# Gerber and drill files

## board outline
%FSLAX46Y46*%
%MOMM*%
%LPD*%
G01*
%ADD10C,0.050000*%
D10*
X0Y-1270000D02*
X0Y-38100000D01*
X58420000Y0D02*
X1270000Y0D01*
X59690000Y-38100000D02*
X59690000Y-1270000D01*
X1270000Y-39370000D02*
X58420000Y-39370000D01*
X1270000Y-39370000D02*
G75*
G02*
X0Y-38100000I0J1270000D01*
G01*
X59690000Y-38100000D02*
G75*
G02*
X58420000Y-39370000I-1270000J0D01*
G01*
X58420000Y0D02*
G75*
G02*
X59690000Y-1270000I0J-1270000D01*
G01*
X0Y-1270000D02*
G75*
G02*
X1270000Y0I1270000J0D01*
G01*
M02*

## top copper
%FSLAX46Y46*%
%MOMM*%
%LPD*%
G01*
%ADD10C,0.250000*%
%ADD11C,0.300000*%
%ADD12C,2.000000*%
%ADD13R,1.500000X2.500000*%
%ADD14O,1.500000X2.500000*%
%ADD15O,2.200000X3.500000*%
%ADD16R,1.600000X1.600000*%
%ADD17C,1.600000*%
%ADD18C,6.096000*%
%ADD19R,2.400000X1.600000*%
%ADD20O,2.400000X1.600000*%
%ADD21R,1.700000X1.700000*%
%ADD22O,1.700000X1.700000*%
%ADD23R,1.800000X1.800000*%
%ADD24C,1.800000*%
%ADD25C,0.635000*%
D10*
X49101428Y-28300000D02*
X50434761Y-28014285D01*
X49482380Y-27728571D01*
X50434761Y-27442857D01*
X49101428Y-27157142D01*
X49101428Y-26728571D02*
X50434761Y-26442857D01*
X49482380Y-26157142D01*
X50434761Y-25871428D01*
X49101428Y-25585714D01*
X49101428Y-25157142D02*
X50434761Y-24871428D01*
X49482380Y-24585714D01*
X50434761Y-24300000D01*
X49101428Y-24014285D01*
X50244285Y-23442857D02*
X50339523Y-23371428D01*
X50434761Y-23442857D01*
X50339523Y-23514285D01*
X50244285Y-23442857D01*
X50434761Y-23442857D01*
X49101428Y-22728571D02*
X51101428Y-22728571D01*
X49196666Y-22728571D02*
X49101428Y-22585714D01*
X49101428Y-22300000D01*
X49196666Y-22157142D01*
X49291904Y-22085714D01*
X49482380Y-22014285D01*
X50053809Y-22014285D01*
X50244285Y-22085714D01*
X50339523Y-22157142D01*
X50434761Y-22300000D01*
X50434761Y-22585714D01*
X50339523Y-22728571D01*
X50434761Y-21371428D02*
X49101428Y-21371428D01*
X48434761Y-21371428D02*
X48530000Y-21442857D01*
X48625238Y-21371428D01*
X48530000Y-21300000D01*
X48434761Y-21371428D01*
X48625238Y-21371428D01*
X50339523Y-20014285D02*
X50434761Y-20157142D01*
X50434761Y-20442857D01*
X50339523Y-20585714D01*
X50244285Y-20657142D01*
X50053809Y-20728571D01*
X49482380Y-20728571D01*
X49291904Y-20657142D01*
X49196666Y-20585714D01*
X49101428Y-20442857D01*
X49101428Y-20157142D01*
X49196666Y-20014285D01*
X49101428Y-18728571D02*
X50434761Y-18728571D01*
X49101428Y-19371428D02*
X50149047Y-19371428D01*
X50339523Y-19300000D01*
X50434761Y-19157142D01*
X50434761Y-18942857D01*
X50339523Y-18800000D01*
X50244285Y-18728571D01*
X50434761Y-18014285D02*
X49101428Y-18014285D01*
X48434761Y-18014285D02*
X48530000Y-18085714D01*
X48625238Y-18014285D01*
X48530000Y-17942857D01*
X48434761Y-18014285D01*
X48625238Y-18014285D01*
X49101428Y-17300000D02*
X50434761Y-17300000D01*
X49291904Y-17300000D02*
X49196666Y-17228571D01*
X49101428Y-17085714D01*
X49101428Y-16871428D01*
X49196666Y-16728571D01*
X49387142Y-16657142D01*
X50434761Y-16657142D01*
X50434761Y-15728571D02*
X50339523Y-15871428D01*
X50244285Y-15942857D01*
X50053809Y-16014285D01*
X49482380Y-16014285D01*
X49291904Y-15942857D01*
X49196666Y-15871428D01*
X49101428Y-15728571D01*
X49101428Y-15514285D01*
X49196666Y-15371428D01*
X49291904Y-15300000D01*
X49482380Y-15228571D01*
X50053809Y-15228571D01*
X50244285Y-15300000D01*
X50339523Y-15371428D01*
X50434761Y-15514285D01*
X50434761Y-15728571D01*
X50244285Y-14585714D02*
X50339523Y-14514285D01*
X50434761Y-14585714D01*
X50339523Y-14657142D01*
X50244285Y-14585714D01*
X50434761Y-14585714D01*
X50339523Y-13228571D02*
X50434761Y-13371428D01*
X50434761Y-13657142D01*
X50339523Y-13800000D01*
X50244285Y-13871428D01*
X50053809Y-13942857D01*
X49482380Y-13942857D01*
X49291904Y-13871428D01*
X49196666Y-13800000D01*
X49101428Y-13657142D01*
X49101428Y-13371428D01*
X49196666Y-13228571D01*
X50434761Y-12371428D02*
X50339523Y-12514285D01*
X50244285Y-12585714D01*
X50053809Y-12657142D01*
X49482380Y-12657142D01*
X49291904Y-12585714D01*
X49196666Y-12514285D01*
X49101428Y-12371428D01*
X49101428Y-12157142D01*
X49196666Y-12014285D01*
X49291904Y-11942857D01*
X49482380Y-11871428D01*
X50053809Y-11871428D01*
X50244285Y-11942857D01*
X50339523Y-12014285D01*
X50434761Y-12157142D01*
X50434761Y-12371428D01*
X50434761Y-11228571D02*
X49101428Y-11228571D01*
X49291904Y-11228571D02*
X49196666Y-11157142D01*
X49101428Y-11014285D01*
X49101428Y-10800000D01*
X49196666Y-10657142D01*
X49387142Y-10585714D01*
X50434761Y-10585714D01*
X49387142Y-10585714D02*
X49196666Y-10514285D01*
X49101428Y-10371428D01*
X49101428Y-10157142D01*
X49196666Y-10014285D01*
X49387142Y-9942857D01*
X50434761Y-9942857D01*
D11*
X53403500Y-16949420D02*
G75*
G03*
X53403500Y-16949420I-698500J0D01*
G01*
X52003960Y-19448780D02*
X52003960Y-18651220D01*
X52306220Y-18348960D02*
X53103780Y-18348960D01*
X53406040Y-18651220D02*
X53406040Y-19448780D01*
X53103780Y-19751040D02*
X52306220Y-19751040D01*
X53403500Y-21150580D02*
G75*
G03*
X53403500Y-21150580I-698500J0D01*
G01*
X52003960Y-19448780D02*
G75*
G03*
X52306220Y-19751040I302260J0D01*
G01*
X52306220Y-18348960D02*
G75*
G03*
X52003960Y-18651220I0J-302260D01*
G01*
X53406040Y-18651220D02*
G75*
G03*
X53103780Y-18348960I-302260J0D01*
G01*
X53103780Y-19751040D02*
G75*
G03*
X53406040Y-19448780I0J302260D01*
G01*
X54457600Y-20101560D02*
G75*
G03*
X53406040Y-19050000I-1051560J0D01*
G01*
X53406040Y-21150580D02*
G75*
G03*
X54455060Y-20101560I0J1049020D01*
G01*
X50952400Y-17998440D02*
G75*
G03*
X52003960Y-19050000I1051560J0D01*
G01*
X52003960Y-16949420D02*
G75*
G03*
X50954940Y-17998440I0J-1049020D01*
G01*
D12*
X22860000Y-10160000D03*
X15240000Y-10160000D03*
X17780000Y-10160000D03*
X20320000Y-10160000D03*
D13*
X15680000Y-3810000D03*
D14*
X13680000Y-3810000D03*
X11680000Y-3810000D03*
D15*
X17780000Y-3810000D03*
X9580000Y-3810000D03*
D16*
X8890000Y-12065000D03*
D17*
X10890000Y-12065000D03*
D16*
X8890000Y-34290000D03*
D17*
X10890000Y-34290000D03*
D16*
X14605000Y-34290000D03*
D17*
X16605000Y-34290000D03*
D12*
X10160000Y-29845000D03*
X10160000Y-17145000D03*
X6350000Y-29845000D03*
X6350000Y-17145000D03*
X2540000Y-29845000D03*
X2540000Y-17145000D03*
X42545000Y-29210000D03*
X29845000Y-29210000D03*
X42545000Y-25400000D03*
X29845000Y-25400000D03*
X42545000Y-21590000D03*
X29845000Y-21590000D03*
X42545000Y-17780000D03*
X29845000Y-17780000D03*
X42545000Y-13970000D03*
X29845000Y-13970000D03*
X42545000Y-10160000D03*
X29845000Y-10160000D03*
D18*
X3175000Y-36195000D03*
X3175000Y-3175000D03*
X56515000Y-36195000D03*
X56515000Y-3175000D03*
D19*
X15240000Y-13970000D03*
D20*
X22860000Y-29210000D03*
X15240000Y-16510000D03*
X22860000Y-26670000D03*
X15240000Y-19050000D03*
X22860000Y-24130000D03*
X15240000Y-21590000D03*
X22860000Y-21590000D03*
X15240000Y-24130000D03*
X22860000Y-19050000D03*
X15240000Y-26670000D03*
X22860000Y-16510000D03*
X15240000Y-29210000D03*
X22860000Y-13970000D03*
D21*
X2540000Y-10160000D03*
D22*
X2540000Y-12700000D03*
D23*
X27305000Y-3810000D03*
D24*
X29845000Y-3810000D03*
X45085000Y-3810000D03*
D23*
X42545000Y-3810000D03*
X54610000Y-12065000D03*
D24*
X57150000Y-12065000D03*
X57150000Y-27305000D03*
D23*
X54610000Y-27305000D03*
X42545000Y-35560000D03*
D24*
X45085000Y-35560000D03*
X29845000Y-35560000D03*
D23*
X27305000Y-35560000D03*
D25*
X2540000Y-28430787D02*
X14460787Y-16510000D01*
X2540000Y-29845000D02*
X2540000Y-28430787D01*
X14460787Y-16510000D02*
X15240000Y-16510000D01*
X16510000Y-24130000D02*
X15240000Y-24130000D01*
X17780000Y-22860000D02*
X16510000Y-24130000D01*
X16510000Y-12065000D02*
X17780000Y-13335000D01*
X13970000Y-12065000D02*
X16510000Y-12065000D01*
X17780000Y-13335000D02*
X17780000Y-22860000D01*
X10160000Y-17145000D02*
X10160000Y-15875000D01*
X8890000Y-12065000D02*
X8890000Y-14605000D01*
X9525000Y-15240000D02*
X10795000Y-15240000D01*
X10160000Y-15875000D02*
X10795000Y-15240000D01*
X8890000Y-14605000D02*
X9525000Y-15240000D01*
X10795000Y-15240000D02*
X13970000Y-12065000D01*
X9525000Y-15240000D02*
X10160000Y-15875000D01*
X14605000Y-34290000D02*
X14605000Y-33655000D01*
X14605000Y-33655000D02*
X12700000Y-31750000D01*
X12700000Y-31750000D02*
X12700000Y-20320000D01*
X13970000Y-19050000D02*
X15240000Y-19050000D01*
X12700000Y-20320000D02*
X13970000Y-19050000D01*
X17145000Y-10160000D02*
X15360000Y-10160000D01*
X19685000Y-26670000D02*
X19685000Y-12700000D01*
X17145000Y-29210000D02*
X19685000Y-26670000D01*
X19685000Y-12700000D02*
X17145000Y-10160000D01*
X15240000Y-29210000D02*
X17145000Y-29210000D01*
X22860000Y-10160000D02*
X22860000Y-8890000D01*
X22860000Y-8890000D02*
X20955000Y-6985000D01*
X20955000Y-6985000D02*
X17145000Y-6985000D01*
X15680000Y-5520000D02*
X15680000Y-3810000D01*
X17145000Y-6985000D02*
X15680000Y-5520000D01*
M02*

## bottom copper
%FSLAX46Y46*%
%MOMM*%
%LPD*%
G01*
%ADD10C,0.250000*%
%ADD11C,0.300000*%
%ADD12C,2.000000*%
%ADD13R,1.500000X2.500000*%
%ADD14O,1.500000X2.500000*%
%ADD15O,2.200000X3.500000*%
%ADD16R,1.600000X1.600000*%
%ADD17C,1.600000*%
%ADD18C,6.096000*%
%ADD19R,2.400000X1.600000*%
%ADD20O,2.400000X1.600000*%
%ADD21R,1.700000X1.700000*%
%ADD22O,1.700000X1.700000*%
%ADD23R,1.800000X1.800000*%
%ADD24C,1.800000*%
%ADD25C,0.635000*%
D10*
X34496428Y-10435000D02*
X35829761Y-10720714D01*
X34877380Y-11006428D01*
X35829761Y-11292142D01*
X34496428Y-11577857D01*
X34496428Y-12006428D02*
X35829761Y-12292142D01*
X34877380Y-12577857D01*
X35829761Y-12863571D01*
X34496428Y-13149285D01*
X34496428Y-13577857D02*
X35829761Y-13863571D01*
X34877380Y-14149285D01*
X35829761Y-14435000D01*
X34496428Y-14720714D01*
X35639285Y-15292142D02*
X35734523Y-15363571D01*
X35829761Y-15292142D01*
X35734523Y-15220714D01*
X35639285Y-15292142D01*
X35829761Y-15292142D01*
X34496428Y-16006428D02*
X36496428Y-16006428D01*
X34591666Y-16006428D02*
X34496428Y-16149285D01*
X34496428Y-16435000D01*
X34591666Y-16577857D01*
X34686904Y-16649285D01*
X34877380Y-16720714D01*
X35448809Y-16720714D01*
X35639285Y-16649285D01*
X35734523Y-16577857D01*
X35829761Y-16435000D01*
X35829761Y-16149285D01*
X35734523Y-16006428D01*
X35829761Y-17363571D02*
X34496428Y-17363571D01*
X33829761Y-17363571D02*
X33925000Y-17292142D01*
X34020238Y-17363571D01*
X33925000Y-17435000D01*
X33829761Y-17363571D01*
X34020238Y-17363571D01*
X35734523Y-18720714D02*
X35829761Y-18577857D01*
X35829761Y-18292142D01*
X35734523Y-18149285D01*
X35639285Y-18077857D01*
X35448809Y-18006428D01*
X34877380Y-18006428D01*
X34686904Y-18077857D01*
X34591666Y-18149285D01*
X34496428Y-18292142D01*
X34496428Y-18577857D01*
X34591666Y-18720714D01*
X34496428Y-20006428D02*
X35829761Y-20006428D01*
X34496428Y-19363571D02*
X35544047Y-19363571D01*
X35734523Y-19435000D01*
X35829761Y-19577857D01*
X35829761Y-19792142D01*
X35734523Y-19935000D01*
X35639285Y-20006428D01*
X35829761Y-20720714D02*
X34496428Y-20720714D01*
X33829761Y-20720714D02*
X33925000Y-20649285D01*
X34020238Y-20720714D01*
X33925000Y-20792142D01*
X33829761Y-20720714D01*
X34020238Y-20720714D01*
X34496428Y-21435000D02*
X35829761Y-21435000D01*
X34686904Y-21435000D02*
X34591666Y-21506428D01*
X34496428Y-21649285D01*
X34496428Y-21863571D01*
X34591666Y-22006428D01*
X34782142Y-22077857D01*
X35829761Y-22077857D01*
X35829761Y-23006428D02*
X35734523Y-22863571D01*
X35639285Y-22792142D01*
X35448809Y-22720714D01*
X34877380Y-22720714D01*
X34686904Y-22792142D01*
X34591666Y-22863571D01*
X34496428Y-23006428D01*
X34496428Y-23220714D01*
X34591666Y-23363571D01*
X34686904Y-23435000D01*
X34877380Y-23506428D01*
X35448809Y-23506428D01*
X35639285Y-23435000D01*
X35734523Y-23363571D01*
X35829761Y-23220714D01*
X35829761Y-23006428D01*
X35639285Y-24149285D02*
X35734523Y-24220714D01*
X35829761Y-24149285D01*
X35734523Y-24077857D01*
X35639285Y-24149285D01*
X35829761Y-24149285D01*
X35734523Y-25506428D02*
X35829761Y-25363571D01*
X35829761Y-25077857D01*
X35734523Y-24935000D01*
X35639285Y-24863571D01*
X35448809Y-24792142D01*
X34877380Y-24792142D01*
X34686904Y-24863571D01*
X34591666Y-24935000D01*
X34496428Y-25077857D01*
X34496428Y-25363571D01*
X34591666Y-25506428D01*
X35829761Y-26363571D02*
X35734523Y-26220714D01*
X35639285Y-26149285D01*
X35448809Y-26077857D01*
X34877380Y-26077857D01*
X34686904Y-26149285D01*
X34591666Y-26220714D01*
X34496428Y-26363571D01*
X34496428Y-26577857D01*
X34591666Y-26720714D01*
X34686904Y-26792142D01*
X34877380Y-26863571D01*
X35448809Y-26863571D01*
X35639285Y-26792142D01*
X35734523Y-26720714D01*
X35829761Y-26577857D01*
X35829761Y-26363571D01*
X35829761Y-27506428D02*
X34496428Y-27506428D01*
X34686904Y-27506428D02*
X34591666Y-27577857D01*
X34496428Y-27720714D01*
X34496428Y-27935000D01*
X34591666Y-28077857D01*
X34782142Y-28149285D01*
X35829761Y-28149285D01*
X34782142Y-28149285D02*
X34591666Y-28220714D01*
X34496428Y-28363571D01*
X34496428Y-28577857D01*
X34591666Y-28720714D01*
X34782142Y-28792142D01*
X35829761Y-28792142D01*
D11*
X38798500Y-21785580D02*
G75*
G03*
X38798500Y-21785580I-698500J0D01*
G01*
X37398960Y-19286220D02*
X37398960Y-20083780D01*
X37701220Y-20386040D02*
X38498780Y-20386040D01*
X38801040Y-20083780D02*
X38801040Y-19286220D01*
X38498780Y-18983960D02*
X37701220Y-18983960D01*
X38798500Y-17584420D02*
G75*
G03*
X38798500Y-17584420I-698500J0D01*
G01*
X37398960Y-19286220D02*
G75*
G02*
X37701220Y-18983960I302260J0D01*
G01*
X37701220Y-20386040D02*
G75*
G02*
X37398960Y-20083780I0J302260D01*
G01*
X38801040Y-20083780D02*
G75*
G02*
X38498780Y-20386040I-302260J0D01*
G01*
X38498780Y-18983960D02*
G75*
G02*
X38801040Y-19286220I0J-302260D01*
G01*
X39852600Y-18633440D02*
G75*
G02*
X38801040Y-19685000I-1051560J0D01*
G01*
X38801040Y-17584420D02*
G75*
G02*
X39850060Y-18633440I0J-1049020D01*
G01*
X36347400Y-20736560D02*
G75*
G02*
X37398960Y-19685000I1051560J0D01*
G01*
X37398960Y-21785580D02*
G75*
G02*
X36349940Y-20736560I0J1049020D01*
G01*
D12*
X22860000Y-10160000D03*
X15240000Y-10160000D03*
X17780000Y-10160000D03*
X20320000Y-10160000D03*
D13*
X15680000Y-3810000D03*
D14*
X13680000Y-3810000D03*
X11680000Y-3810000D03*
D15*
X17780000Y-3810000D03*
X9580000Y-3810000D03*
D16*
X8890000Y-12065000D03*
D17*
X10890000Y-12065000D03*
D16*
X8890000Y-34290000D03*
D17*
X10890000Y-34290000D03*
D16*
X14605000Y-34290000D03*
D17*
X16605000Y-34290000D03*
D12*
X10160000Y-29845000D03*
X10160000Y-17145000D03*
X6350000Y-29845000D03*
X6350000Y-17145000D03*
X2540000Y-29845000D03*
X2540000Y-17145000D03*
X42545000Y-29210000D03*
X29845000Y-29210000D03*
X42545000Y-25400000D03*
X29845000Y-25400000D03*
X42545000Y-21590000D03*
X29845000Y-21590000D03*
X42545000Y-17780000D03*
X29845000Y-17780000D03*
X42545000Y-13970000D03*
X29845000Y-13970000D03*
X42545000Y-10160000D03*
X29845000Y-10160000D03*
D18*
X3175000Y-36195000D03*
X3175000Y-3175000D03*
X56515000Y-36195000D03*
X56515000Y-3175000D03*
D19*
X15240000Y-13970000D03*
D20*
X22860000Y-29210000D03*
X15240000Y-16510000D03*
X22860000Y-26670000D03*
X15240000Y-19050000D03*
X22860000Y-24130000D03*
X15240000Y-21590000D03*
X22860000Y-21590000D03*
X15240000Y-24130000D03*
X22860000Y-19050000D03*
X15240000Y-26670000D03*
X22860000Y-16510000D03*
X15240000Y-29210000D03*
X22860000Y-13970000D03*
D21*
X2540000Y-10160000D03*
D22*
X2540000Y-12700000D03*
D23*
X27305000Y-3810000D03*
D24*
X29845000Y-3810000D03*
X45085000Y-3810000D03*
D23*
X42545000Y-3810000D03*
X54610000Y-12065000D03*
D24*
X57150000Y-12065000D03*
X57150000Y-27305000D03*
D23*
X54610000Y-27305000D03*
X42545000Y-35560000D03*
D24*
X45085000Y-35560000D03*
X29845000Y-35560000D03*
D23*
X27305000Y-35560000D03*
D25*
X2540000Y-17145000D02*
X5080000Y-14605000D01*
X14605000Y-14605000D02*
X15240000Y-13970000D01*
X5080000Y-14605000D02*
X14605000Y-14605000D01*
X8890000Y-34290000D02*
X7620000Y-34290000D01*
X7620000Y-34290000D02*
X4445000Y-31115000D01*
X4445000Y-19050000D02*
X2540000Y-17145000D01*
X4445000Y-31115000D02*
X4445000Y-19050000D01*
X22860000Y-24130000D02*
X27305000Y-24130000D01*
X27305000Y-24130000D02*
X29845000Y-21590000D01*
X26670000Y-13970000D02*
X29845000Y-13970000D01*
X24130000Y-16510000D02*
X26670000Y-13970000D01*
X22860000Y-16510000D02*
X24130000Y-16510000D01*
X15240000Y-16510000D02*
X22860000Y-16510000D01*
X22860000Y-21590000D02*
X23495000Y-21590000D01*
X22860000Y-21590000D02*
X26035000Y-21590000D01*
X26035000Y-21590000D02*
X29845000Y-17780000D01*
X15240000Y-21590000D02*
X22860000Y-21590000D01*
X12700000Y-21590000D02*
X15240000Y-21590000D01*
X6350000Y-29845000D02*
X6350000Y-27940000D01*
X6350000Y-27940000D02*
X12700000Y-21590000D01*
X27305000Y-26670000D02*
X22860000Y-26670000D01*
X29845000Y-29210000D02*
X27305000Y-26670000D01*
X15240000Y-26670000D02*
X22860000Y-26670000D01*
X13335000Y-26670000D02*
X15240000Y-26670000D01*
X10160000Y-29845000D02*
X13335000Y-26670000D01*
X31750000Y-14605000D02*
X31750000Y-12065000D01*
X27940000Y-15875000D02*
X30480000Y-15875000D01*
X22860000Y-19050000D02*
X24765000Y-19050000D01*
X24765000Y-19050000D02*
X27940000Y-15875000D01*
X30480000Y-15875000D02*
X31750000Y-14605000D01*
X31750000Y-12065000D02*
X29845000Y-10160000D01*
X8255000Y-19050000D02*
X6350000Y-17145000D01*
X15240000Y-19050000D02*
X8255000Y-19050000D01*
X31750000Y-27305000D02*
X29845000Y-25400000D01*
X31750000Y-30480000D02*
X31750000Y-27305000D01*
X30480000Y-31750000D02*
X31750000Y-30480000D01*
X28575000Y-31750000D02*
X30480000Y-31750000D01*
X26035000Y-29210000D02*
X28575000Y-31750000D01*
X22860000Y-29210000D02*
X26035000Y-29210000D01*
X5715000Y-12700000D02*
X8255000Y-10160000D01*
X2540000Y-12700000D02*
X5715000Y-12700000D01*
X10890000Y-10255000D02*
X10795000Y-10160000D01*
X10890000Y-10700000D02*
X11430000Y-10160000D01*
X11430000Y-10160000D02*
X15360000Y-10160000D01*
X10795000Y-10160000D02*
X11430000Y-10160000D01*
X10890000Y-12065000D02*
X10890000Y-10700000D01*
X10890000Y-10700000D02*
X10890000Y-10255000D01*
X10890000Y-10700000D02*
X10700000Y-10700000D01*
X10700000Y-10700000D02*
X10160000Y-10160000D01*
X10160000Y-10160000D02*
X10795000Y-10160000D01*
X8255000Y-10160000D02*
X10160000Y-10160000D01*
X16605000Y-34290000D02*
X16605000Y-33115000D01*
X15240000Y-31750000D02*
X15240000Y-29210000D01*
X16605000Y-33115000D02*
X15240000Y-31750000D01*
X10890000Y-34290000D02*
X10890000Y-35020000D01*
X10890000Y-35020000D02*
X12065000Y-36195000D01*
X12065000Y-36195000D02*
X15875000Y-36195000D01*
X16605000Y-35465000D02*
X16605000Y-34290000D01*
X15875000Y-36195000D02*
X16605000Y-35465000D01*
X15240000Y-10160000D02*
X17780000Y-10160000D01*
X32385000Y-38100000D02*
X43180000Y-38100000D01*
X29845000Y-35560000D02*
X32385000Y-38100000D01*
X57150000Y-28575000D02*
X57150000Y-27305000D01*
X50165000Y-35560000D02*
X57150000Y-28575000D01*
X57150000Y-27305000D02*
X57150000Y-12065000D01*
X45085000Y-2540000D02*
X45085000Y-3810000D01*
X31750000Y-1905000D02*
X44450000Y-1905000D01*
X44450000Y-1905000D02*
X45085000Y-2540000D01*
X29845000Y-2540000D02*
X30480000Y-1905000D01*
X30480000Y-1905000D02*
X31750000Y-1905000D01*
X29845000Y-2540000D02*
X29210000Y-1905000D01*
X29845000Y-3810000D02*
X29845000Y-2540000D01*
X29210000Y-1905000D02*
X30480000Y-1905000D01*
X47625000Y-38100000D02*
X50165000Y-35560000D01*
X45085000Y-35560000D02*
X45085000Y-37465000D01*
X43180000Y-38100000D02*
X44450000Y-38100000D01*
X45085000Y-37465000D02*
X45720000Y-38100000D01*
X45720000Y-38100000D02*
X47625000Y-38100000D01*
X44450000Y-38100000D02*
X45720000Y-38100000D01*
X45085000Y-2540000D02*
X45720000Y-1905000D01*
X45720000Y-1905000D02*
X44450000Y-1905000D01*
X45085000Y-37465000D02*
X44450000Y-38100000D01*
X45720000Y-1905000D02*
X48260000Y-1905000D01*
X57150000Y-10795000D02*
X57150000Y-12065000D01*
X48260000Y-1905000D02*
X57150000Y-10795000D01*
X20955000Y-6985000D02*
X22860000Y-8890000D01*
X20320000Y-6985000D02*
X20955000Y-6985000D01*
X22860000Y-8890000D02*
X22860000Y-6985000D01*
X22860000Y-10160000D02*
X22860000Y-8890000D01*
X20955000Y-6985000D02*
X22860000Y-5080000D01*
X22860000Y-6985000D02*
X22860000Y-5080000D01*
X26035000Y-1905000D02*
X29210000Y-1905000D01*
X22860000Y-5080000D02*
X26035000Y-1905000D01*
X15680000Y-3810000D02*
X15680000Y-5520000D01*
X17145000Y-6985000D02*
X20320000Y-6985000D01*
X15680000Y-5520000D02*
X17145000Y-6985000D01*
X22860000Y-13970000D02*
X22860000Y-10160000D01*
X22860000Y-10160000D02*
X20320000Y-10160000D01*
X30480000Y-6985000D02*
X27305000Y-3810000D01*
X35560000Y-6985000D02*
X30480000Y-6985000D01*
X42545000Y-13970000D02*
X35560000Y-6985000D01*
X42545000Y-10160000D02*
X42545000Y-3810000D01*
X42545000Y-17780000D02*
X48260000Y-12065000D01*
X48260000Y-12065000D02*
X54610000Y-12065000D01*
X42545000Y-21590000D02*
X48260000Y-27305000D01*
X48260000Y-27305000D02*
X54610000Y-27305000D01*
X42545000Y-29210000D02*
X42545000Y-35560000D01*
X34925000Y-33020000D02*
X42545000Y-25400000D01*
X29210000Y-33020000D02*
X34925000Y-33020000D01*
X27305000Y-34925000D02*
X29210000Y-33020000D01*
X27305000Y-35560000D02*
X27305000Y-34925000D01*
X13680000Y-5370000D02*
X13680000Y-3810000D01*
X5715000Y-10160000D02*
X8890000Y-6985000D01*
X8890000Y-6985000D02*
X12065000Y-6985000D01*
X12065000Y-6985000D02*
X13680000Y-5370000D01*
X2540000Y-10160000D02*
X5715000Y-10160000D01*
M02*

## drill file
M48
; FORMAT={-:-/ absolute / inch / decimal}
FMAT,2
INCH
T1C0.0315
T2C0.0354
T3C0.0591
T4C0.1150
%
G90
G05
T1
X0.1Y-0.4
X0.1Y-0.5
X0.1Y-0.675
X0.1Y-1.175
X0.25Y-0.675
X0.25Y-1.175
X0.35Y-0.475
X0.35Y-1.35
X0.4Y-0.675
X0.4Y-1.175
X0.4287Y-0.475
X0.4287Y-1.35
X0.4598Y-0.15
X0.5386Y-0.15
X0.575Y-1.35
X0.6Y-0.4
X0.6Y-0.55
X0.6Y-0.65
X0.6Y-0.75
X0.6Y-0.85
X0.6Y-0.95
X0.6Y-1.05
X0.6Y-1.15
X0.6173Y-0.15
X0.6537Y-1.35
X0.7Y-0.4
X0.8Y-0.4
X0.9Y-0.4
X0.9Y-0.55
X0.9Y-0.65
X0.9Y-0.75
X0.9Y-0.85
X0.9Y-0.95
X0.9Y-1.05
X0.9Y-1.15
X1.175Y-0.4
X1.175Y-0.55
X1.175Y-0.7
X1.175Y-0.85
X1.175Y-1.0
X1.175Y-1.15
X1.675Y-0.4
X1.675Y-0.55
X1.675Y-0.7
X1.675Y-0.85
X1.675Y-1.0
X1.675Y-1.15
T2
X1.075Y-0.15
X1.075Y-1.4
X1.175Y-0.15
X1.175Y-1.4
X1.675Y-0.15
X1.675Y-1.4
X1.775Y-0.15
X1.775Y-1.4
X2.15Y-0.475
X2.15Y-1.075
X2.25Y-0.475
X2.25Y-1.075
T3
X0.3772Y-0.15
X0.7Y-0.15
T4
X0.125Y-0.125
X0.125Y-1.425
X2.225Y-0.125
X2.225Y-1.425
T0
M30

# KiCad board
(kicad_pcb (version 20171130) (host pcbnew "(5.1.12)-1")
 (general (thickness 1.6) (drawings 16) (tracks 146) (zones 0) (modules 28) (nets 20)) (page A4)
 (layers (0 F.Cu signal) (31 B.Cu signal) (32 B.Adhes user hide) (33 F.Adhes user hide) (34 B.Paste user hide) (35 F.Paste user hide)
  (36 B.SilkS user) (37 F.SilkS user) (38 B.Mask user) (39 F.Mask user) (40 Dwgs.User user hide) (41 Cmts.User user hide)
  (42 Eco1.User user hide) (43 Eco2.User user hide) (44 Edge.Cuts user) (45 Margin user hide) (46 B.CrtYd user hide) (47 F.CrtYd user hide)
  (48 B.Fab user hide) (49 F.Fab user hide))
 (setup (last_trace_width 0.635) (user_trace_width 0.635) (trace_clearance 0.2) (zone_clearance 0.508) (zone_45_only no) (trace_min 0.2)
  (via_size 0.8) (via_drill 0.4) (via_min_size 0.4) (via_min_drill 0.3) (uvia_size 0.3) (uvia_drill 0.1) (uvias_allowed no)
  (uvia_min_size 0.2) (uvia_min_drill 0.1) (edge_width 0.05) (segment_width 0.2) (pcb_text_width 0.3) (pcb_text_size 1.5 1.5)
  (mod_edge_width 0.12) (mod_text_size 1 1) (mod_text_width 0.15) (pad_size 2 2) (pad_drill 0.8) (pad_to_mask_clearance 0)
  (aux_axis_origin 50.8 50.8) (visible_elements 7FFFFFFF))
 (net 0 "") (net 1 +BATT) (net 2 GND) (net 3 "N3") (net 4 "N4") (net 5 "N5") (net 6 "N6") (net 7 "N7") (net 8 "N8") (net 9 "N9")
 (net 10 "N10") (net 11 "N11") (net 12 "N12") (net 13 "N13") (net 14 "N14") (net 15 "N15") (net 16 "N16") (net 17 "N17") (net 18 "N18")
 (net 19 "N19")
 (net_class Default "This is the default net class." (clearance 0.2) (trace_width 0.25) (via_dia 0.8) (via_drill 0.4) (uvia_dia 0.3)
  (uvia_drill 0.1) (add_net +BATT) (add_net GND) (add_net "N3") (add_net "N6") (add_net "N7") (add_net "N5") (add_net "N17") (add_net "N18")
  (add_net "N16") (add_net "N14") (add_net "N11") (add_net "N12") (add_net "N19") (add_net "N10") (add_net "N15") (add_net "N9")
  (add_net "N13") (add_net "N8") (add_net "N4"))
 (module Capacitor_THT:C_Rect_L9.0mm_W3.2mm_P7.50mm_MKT (layer F.Cu) (at 73.66 60.96 180)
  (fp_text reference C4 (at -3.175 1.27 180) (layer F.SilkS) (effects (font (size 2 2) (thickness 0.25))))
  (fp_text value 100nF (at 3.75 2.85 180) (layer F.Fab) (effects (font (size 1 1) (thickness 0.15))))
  (pad 1 thru_hole circle (at 0 0 180) (size 2 2) (drill 0.8) (layers *.Cu *.Mask) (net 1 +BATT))
  (pad 2 thru_hole circle (at 7.62 0 180) (size 2 2) (drill 0.8) (layers *.Cu *.Mask) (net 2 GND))
  (pad 2 thru_hole circle (at 5.08 0 180) (size 2 2) (drill 0.8) (layers *.Cu *.Mask) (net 2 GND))
  (pad 1 thru_hole circle (at 2.54 0 180) (size 2 2) (drill 0.8) (layers *.Cu *.Mask) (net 1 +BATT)))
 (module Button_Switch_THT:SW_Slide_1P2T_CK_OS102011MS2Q (layer F.Cu) (at 66.48 54.61 180)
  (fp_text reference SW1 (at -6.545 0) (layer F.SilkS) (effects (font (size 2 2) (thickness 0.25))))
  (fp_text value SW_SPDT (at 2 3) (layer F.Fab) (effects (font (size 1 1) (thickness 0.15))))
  (pad 1 thru_hole rect (at 0 0 180) (size 1.5 2.5) (drill 0.8) (layers *.Cu *.Mask) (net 1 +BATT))
  (pad 2 thru_hole oval (at 2 0 180) (size 1.5 2.5) (drill 0.8) (layers *.Cu *.Mask) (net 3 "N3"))
  (pad 3 thru_hole oval (at 4 0 180) (size 1.5 2.5) (drill 0.8) (layers *.Cu *.Mask) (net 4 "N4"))
  (pad "" thru_hole oval (at -2.1 0 180) (size 2.2 3.5) (drill 1.5) (layers *.Cu *.Mask))
  (pad "" thru_hole oval (at 6.1 0 180) (size 2.2 3.5) (drill 1.5) (layers *.Cu *.Mask)))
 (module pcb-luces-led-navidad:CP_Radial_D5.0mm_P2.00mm (layer F.Cu) (at 59.69 62.865)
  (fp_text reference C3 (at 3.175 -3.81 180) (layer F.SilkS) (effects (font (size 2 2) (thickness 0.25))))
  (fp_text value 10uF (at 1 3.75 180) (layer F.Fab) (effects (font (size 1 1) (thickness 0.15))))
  (pad 1 thru_hole rect (at 0 0) (size 1.6 1.6) (drill 0.8) (layers *.Cu *.Mask) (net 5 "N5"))
  (pad 2 thru_hole circle (at 2 0) (size 1.6 1.6) (drill 0.8) (layers *.Cu *.Mask) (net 2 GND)))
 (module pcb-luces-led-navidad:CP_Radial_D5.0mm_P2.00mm (layer F.Cu) (at 59.69 85.09)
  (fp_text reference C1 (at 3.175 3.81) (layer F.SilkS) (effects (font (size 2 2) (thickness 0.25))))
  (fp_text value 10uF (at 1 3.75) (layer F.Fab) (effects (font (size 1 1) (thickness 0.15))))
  (pad 1 thru_hole rect (at 0 0) (size 1.6 1.6) (drill 0.8) (layers *.Cu *.Mask) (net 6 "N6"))
  (pad 2 thru_hole circle (at 2 0) (size 1.6 1.6) (drill 0.8) (layers *.Cu *.Mask) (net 2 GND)))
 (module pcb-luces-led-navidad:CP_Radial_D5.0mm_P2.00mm (layer F.Cu) (at 65.405 85.09)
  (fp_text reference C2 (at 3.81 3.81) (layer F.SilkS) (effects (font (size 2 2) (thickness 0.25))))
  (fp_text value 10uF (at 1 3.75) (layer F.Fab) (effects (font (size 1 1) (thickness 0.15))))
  (pad 1 thru_hole rect (at 0 0) (size 1.6 1.6) (drill 0.8) (layers *.Cu *.Mask) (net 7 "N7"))
  (pad 2 thru_hole circle (at 2 0) (size 1.6 1.6) (drill 0.8) (layers *.Cu *.Mask) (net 2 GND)))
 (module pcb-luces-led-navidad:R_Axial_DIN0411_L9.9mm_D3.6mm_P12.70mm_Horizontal (layer F.Cu) (at 60.96 80.645 90)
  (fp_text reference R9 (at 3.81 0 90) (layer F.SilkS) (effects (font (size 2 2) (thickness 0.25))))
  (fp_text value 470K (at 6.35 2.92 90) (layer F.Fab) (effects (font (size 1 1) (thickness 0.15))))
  (pad 1 thru_hole circle (at 0 0 90) (size 2 2) (drill 0.8) (layers *.Cu *.Mask) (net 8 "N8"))
  (pad 2 thru_hole circle (at 12.7 0 90) (size 2 2) (drill 0.8) (layers *.Cu *.Mask) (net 5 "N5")))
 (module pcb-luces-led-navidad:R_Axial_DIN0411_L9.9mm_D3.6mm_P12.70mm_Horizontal (layer F.Cu) (at 57.15 80.645 90)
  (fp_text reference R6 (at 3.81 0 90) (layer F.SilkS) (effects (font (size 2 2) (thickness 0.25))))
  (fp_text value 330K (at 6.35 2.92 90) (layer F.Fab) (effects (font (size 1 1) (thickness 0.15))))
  (pad 1 thru_hole circle (at 0 0 90) (size 2 2) (drill 0.8) (layers *.Cu *.Mask) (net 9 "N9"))
  (pad 2 thru_hole circle (at 12.7 0 90) (size 2 2) (drill 0.8) (layers *.Cu *.Mask) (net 7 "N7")))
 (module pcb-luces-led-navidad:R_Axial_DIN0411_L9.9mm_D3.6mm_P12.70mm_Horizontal (layer F.Cu) (at 53.34 80.645 90)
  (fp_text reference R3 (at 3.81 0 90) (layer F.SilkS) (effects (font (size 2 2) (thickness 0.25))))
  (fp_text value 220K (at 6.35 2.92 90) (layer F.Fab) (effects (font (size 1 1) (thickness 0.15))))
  (pad 1 thru_hole circle (at 0 0 90) (size 2 2) (drill 0.8) (layers *.Cu *.Mask) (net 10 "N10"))
  (pad 2 thru_hole circle (at 12.7 0 90) (size 2 2) (drill 0.8) (layers *.Cu *.Mask) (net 6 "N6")))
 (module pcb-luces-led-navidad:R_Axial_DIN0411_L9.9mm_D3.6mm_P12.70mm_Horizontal (layer F.Cu) (at 93.345 80.01 180)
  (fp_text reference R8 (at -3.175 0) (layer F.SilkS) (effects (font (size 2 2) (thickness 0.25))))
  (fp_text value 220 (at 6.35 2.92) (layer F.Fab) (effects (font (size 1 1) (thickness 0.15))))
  (pad 1 thru_hole circle (at 0 0 180) (size 2 2) (drill 0.8) (layers *.Cu *.Mask) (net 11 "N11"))
  (pad 2 thru_hole circle (at 12.7 0 180) (size 2 2) (drill 0.8) (layers *.Cu *.Mask) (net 8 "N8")))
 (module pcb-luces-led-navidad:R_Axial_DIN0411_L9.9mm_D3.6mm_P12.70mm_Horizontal (layer F.Cu) (at 93.345 76.2 180)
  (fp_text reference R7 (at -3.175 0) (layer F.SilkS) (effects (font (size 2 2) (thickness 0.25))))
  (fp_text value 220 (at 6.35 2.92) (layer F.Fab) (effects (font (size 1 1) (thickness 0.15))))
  (pad 1 thru_hole circle (at 0 0 180) (size 2 2) (drill 0.8) (layers *.Cu *.Mask) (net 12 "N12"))
  (pad 2 thru_hole circle (at 12.7 0 180) (size 2 2) (drill 0.8) (layers *.Cu *.Mask) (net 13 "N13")))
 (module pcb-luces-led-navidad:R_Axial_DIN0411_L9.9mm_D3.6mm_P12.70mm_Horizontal (layer F.Cu) (at 93.345 72.39 180)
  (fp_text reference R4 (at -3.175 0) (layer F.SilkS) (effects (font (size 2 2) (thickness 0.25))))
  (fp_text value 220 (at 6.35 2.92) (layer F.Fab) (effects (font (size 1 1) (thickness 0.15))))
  (pad 1 thru_hole circle (at 0 0 180) (size 2 2) (drill 0.8) (layers *.Cu *.Mask) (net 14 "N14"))
  (pad 2 thru_hole circle (at 12.7 0 180) (size 2 2) (drill 0.8) (layers *.Cu *.Mask) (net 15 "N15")))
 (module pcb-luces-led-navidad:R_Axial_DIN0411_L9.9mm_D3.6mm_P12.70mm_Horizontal (layer F.Cu) (at 93.345 68.58 180)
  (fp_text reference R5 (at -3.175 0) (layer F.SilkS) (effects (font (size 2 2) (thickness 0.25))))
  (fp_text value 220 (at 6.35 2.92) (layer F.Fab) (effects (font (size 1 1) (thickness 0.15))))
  (pad 1 thru_hole circle (at 0 0 180) (size 2 2) (drill 0.8) (layers *.Cu *.Mask) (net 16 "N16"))
  (pad 2 thru_hole circle (at 12.7 0 180) (size 2 2) (drill 0.8) (layers *.Cu *.Mask) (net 9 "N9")))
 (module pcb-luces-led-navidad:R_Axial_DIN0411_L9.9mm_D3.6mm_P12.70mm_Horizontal (layer F.Cu) (at 93.345 64.77 180)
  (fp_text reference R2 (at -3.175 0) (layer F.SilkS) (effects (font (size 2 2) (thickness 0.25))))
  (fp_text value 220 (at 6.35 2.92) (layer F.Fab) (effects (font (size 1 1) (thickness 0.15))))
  (pad 1 thru_hole circle (at 0 0 180) (size 2 2) (drill 0.8) (layers *.Cu *.Mask) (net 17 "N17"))
  (pad 2 thru_hole circle (at 12.7 0 180) (size 2 2) (drill 0.8) (layers *.Cu *.Mask) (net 10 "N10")))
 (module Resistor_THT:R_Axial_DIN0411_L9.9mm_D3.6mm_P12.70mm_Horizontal (layer F.Cu) (at 93.345 60.96 180)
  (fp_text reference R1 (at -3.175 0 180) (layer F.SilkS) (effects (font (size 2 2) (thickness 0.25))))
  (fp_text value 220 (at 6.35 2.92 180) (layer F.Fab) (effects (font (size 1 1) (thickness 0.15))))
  (pad 1 thru_hole circle (at 0 0 180) (size 2 2) (drill 0.8) (layers *.Cu *.Mask) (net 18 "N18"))
  (pad 2 thru_hole circle (at 12.7 0 180) (size 2 2) (drill 0.8) (layers *.Cu *.Mask) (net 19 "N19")))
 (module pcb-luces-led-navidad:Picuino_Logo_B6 (layer B.Cu) (at 103.505 69.85 270)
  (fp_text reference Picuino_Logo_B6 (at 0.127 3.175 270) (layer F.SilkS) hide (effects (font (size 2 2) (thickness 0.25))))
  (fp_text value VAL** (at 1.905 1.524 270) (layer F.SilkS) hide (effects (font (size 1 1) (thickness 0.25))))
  (fp_circle (center -2.10058 0) (end -1.40208 0) (layer F.Cu) (width 0.3))
  (fp_line (start 0.39878 0.70104) (end -0.39878 0.70104) (layer F.Cu) (width 0.3))
  (fp_line (start -0.70104 0.39878) (end -0.70104 -0.39878) (layer F.Cu) (width 0.3))
  (fp_line (start -0.39878 -0.70104) (end 0.39878 -0.70104) (layer F.Cu) (width 0.3))
  (fp_line (start 0.70104 -0.39878) (end 0.70104 0.39878) (layer F.Cu) (width 0.3))
  (fp_circle (center 2.10058 0) (end 2.79908 0) (layer F.Cu) (width 0.3))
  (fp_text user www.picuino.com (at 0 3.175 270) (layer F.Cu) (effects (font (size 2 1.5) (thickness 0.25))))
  (fp_arc (start 0.39878 0.39878) (end 0.70104 0.39878) (angle 90) (layer F.Cu) (width 0.3))
  (fp_arc (start -0.39878 0.39878) (end -0.39878 0.70104) (angle 90) (layer F.Cu) (width 0.3))
  (fp_arc (start -0.39878 -0.39878) (end -0.70104 -0.39878) (angle 90) (layer F.Cu) (width 0.3))
  (fp_arc (start 0.39878 -0.39878) (end 0.39878 -0.70104) (angle 90) (layer F.Cu) (width 0.3))
  (fp_arc (start 1.05156 -0.70104) (end 0 -0.70104) (angle 90) (layer F.Cu) (width 0.3))
  (fp_arc (start 1.05156 -0.70104) (end 1.05156 -1.75006) (angle 90) (layer F.Cu) (width 0.3))
  (fp_arc (start -1.05156 0.70104) (end 0 0.70104) (angle 90) (layer F.Cu) (width 0.3))
  (fp_arc (start -1.05156 0.70104) (end -1.05156 1.75006) (angle 90) (layer F.Cu) (width 0.3)))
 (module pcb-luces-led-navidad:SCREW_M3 (layer F.Cu) (at 53.975 86.995)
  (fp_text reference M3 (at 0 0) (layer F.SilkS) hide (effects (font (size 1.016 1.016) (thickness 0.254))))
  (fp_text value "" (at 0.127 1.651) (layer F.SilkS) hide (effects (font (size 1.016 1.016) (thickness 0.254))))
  (pad "" thru_hole circle (at 0 0) (size 6.096 6.096) (drill 2.921) (layers *.Cu F.SilkS)))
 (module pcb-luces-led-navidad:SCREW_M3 (layer F.Cu) (at 53.975 53.975)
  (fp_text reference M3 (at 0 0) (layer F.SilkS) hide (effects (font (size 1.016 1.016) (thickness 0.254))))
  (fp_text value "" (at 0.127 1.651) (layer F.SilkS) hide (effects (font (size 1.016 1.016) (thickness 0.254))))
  (pad "" thru_hole circle (at 0 0) (size 6.096 6.096) (drill 2.921) (layers *.Cu F.SilkS)))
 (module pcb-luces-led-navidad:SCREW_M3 (layer F.Cu) (at 107.315 86.995)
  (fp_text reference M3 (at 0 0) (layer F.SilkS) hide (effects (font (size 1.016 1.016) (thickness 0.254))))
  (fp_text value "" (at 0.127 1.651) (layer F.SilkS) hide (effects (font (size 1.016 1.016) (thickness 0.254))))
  (pad "" thru_hole circle (at 0 0) (size 6.096 6.096) (drill 2.921) (layers *.Cu F.SilkS)))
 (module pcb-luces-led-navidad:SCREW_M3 (layer F.Cu) (at 107.315 53.975)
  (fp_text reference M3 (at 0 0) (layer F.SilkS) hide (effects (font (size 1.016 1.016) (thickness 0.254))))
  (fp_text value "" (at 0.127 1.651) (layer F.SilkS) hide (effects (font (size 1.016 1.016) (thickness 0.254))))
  (pad "" thru_hole circle (at 0 0) (size 6.096 6.096) (drill 2.921) (layers *.Cu F.SilkS)))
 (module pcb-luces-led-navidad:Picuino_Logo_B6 (layer F.Cu) (at 88.9 70.485 90)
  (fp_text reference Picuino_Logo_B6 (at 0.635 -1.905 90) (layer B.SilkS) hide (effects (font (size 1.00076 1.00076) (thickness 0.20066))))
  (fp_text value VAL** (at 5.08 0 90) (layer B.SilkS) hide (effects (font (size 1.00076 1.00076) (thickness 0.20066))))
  (fp_circle (center -2.10058 0) (end -1.40208 0) (layer B.Cu) (width 0.3))
  (fp_line (start 0.39878 -0.70104) (end -0.39878 -0.70104) (layer B.Cu) (width 0.3))
  (fp_line (start -0.70104 -0.39878) (end -0.70104 0.39878) (layer B.Cu) (width 0.3))
  (fp_line (start -0.39878 0.70104) (end 0.39878 0.70104) (layer B.Cu) (width 0.3))
  (fp_line (start 0.70104 0.39878) (end 0.70104 -0.39878) (layer B.Cu) (width 0.3))
  (fp_circle (center 2.10058 0) (end 2.79908 0) (layer B.Cu) (width 0.3))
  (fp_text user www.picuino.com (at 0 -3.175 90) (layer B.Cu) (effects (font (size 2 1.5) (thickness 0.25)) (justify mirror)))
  (fp_arc (start 0.39878 -0.39878) (end 0.70104 -0.39878) (angle -90) (layer B.Cu) (width 0.3))
  (fp_arc (start -0.39878 -0.39878) (end -0.39878 -0.70104) (angle -90) (layer B.Cu) (width 0.3))
  (fp_arc (start -0.39878 0.39878) (end -0.70104 0.39878) (angle -90) (layer B.Cu) (width 0.3))
  (fp_arc (start 0.39878 0.39878) (end 0.39878 0.70104) (angle -90) (layer B.Cu) (width 0.3))
  (fp_arc (start 1.05156 0.70104) (end 0 0.70104) (angle -90) (layer B.Cu) (width 0.3))
  (fp_arc (start 1.05156 0.70104) (end 1.05156 1.75006) (angle -90) (layer B.Cu) (width 0.3))
  (fp_arc (start -1.05156 -0.70104) (end 0 -0.70104) (angle -90) (layer B.Cu) (width 0.3))
  (fp_arc (start -1.05156 -0.70104) (end -1.05156 -1.75006) (angle -90) (layer B.Cu) (width 0.3)))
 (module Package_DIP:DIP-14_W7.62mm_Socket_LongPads (layer F.Cu) (at 66.04 64.77)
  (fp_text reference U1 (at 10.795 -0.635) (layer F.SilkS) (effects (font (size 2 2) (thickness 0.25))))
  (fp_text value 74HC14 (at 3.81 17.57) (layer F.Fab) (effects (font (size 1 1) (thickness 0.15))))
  (pad 1 thru_hole rect (at 0 0) (size 2.4 1.6) (drill 0.8) (layers *.Cu *.Mask) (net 6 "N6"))
  (pad 8 thru_hole oval (at 7.62 15.24) (size 2.4 1.6) (drill 0.8) (layers *.Cu *.Mask) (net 13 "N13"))
  (pad 2 thru_hole oval (at 0 2.54) (size 2.4 1.6) (drill 0.8) (layers *.Cu *.Mask) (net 10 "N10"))
  (pad 9 thru_hole oval (at 7.62 12.7) (size 2.4 1.6) (drill 0.8) (layers *.Cu *.Mask) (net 8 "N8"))
  (pad 3 thru_hole oval (at 0 5.08) (size 2.4 1.6) (drill 0.8) (layers *.Cu *.Mask) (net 7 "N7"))
  (pad 10 thru_hole oval (at 7.62 10.16) (size 2.4 1.6) (drill 0.8) (layers *.Cu *.Mask) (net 15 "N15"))
  (pad 4 thru_hole oval (at 0 7.62) (size 2.4 1.6) (drill 0.8) (layers *.Cu *.Mask) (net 9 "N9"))
  (pad 11 thru_hole oval (at 7.62 7.62) (size 2.4 1.6) (drill 0.8) (layers *.Cu *.Mask) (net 9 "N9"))
  (pad 5 thru_hole oval (at 0 10.16) (size 2.4 1.6) (drill 0.8) (layers *.Cu *.Mask) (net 5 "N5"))
  (pad 12 thru_hole oval (at 7.62 5.08) (size 2.4 1.6) (drill 0.8) (layers *.Cu *.Mask) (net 19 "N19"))
  (pad 6 thru_hole oval (at 0 12.7) (size 2.4 1.6) (drill 0.8) (layers *.Cu *.Mask) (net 8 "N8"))
  (pad 13 thru_hole oval (at 7.62 2.54) (size 2.4 1.6) (drill 0.8) (layers *.Cu *.Mask) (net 10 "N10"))
  (pad 7 thru_hole oval (at 0 15.24) (size 2.4 1.6) (drill 0.8) (layers *.Cu *.Mask) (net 2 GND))
  (pad 14 thru_hole oval (at 7.62 0) (size 2.4 1.6) (drill 0.8) (layers *.Cu *.Mask) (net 1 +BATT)))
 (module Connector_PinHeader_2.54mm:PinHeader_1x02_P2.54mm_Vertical (layer F.Cu) (at 53.34 60.96)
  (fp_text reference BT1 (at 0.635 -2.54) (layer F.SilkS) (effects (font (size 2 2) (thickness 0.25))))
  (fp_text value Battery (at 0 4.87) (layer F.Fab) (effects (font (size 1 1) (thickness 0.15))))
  (pad 1 thru_hole rect (at 0 0) (size 1.7 1.7) (drill 0.8) (layers *.Cu *.Mask) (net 3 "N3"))
  (pad 2 thru_hole oval (at 0 2.54) (size 1.7 1.7) (drill 0.8) (layers *.Cu *.Mask) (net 2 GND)))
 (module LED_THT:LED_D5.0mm (layer F.Cu) (at 78.105 54.61)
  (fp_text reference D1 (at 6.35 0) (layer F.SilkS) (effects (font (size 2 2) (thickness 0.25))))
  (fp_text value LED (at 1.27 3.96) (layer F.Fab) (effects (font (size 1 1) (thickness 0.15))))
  (pad 1 thru_hole rect (at 0 0) (size 1.8 1.8) (drill 0.9) (layers *.Cu *.Mask) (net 17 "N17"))
  (pad 2 thru_hole circle (at 2.54 0) (size 1.8 1.8) (drill 0.9) (layers *.Cu *.Mask) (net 1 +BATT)))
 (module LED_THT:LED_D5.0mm (layer F.Cu) (at 93.345 54.61)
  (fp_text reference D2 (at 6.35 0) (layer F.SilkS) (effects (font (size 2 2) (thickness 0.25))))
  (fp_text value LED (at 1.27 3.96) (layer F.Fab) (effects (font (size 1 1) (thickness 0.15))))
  (pad 2 thru_hole circle (at 2.54 0) (size 1.8 1.8) (drill 0.9) (layers *.Cu *.Mask) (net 1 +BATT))
  (pad 1 thru_hole rect (at 0 0) (size 1.8 1.8) (drill 0.9) (layers *.Cu *.Mask) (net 18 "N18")))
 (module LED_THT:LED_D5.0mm (layer F.Cu) (at 105.41 62.865)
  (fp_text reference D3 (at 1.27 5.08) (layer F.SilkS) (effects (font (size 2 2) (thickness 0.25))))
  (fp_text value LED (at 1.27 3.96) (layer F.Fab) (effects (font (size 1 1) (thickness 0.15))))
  (pad 1 thru_hole rect (at 0 0) (size 1.8 1.8) (drill 0.9) (layers *.Cu *.Mask) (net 16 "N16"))
  (pad 2 thru_hole circle (at 2.54 0) (size 1.8 1.8) (drill 0.9) (layers *.Cu *.Mask) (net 1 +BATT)))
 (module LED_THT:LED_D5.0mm (layer F.Cu) (at 105.41 78.105)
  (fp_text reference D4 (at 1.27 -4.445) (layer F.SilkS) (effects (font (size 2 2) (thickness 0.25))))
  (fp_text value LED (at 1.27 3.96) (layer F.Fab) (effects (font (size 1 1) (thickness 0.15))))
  (pad 2 thru_hole circle (at 2.54 0) (size 1.8 1.8) (drill 0.9) (layers *.Cu *.Mask) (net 1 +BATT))
  (pad 1 thru_hole rect (at 0 0) (size 1.8 1.8) (drill 0.9) (layers *.Cu *.Mask) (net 14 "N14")))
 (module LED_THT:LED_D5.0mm (layer F.Cu) (at 93.345 86.36)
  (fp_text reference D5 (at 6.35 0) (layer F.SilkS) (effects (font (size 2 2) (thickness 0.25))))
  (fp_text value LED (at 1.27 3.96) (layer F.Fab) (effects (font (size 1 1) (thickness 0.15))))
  (pad 1 thru_hole rect (at 0 0) (size 1.8 1.8) (drill 0.9) (layers *.Cu *.Mask) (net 11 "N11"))
  (pad 2 thru_hole circle (at 2.54 0) (size 1.8 1.8) (drill 0.9) (layers *.Cu *.Mask) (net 1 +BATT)))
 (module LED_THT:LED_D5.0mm (layer F.Cu) (at 78.105 86.36)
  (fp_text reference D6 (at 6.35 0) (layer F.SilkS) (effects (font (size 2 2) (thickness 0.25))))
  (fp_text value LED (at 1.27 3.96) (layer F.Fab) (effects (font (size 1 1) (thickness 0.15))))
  (pad 2 thru_hole circle (at 2.54 0) (size 1.8 1.8) (drill 0.9) (layers *.Cu *.Mask) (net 1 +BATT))
  (pad 1 thru_hole rect (at 0 0) (size 1.8 1.8) (drill 0.9) (layers *.Cu *.Mask) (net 12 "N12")))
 (gr_line (start 50.8 52.07) (end 50.8 88.9) (layer Edge.Cuts) (width 0.05))
 (gr_line (start 109.22 50.8) (end 52.07 50.8) (layer Edge.Cuts) (width 0.05))
 (gr_line (start 110.49 88.9) (end 110.49 52.07) (layer Edge.Cuts) (width 0.05))
 (gr_line (start 52.07 90.17) (end 109.22 90.17) (layer Edge.Cuts) (width 0.05))
 (gr_arc (start 52.07 88.9) (end 50.8 88.9) (angle -90) (layer Edge.Cuts) (width 0.05))
 (gr_arc (start 109.22 88.9) (end 109.22 90.17) (angle -90) (layer Edge.Cuts) (width 0.05))
 (gr_arc (start 109.22 52.07) (end 110.49 52.07) (angle -90) (layer Edge.Cuts) (width 0.05))
 (gr_arc (start 52.07 52.07) (end 52.07 50.8) (angle -90) (layer Edge.Cuts) (width 0.05))
 (segment (start 53.34 67.945) (end 55.88 65.405) (width 0.635) (layer B.Cu) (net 6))
 (segment (start 65.405 65.405) (end 66.04 64.77) (width 0.635) (layer B.Cu) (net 6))
 (segment (start 55.88 65.405) (end 65.405 65.405) (width 0.635) (layer B.Cu) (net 6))
 (segment (start 59.69 85.09) (end 58.42 85.09) (width 0.635) (layer B.Cu) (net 6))
 (segment (start 58.42 85.09) (end 55.245 81.915) (width 0.635) (layer B.Cu) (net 6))
 (segment (start 55.245 69.85) (end 53.34 67.945) (width 0.635) (layer B.Cu) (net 6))
 (segment (start 55.245 81.915) (end 55.245 69.85) (width 0.635) (layer B.Cu) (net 6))
 (segment (start 73.66 74.93) (end 78.105 74.93) (width 0.635) (layer B.Cu) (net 15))
 (segment (start 78.105 74.93) (end 80.645 72.39) (width 0.635) (layer B.Cu) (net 15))
 (segment (start 77.47 64.77) (end 80.645 64.77) (width 0.635) (layer B.Cu) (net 10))
 (segment (start 74.93 67.31) (end 77.47 64.77) (width 0.635) (layer B.Cu) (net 10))
 (segment (start 73.66 67.31) (end 74.93 67.31) (width 0.635) (layer B.Cu) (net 10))
 (segment (start 66.04 67.31) (end 73.66 67.31) (width 0.635) (layer B.Cu) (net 10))
 (segment (start 53.34 79.230787) (end 65.260787 67.31) (width 0.635) (layer F.Cu) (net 10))
 (segment (start 53.34 80.645) (end 53.34 79.230787) (width 0.635) (layer F.Cu) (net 10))
 (segment (start 65.260787 67.31) (end 66.04 67.31) (width 0.635) (layer F.Cu) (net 10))
 (segment (start 73.66 72.39) (end 74.295 72.39) (width 0.635) (layer B.Cu) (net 9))
 (segment (start 73.66 72.39) (end 76.835 72.39) (width 0.635) (layer B.Cu) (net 9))
 (segment (start 76.835 72.39) (end 80.645 68.58) (width 0.635) (layer B.Cu) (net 9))
 (segment (start 66.04 72.39) (end 73.66 72.39) (width 0.635) (layer B.Cu) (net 9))
 (segment (start 63.5 72.39) (end 66.04 72.39) (width 0.635) (layer B.Cu) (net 9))
 (segment (start 57.15 80.645) (end 57.15 78.74) (width 0.635) (layer B.Cu) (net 9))
 (segment (start 57.15 78.74) (end 63.5 72.39) (width 0.635) (layer B.Cu) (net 9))
 (segment (start 78.105 77.47) (end 73.66 77.47) (width 0.635) (layer B.Cu) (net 8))
 (segment (start 80.645 80.01) (end 78.105 77.47) (width 0.635) (layer B.Cu) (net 8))
 (segment (start 66.04 77.47) (end 73.66 77.47) (width 0.635) (layer B.Cu) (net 8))
 (segment (start 64.135 77.47) (end 66.04 77.47) (width 0.635) (layer B.Cu) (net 8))
 (segment (start 60.96 80.645) (end 64.135 77.47) (width 0.635) (layer B.Cu) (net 8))
 (segment (start 82.55 65.405) (end 82.55 62.865) (width 0.635) (layer B.Cu) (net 19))
 (segment (start 78.74 66.675) (end 81.28 66.675) (width 0.635) (layer B.Cu) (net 19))
 (segment (start 73.66 69.85) (end 75.565 69.85) (width 0.635) (layer B.Cu) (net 19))
 (segment (start 75.565 69.85) (end 78.74 66.675) (width 0.635) (layer B.Cu) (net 19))
 (segment (start 81.28 66.675) (end 82.55 65.405) (width 0.635) (layer B.Cu) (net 19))
 (segment (start 82.55 62.865) (end 80.645 60.96) (width 0.635) (layer B.Cu) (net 19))
 (segment (start 67.31 74.93) (end 66.04 74.93) (width 0.635) (layer F.Cu) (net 5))
 (segment (start 68.58 73.66) (end 67.31 74.93) (width 0.635) (layer F.Cu) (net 5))
 (segment (start 67.31 62.865) (end 68.58 64.135) (width 0.635) (layer F.Cu) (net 5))
 (segment (start 64.77 62.865) (end 67.31 62.865) (width 0.635) (layer F.Cu) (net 5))
 (segment (start 68.58 64.135) (end 68.58 73.66) (width 0.635) (layer F.Cu) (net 5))
 (segment (start 60.96 67.945) (end 60.96 66.675) (width 0.635) (layer F.Cu) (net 5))
 (segment (start 59.69 62.865) (end 59.69 65.405) (width 0.635) (layer F.Cu) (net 5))
 (segment (start 60.325 66.04) (end 61.595 66.04) (width 0.635) (layer F.Cu) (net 5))
 (segment (start 60.96 66.675) (end 61.595 66.04) (width 0.635) (layer F.Cu) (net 5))
 (segment (start 59.69 65.405) (end 60.325 66.04) (width 0.635) (layer F.Cu) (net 5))
 (segment (start 61.595 66.04) (end 64.77 62.865) (width 0.635) (layer F.Cu) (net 5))
 (segment (start 60.325 66.04) (end 60.96 66.675) (width 0.635) (layer F.Cu) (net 5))
 (segment (start 59.055 69.85) (end 57.15 67.945) (width 0.635) (layer B.Cu) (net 7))
 (segment (start 66.04 69.85) (end 59.055 69.85) (width 0.635) (layer B.Cu) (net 7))
 (segment (start 65.405 85.09) (end 65.405 84.455) (width 0.635) (layer F.Cu) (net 7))
 (segment (start 65.405 84.455) (end 63.5 82.55) (width 0.635) (layer F.Cu) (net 7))
 (segment (start 63.5 82.55) (end 63.5 71.12) (width 0.635) (layer F.Cu) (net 7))
 (segment (start 64.77 69.85) (end 66.04 69.85) (width 0.635) (layer F.Cu) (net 7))
 (segment (start 63.5 71.12) (end 64.77 69.85) (width 0.635) (layer F.Cu) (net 7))
 (segment (start 82.55 78.105) (end 80.645 76.2) (width 0.635) (layer B.Cu) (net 13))
 (segment (start 82.55 81.28) (end 82.55 78.105) (width 0.635) (layer B.Cu) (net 13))
 (segment (start 81.28 82.55) (end 82.55 81.28) (width 0.635) (layer B.Cu) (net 13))
 (segment (start 79.375 82.55) (end 81.28 82.55) (width 0.635) (layer B.Cu) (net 13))
 (segment (start 76.835 80.01) (end 79.375 82.55) (width 0.635) (layer B.Cu) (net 13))
 (segment (start 73.66 80.01) (end 76.835 80.01) (width 0.635) (layer B.Cu) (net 13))
 (segment (start 67.945 60.96) (end 66.16 60.96) (width 0.635) (layer F.Cu) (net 2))
 (segment (start 70.485 77.47) (end 70.485 63.5) (width 0.635) (layer F.Cu) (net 2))
 (segment (start 67.945 80.01) (end 70.485 77.47) (width 0.635) (layer F.Cu) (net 2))
 (segment (start 70.485 63.5) (end 67.945 60.96) (width 0.635) (layer F.Cu) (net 2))
 (segment (start 66.04 80.01) (end 67.945 80.01) (width 0.635) (layer F.Cu) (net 2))
 (segment (start 56.515 63.5) (end 59.055 60.96) (width 0.635) (layer B.Cu) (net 2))
 (segment (start 53.34 63.5) (end 56.515 63.5) (width 0.635) (layer B.Cu) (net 2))
 (segment (start 61.69 61.055) (end 61.595 60.96) (width 0.635) (layer B.Cu) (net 2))
 (segment (start 61.69 61.5) (end 62.23 60.96) (width 0.635) (layer B.Cu) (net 2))
 (segment (start 62.23 60.96) (end 66.16 60.96) (width 0.635) (layer B.Cu) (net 2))
 (segment (start 61.595 60.96) (end 62.23 60.96) (width 0.635) (layer B.Cu) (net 2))
 (segment (start 61.69 62.865) (end 61.69 61.5) (width 0.635) (layer B.Cu) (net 2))
 (segment (start 61.69 61.5) (end 61.69 61.055) (width 0.635) (layer B.Cu) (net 2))
 (segment (start 61.69 61.5) (end 61.5 61.5) (width 0.635) (layer B.Cu) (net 2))
 (segment (start 61.5 61.5) (end 60.96 60.96) (width 0.635) (layer B.Cu) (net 2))
 (segment (start 60.96 60.96) (end 61.595 60.96) (width 0.635) (layer B.Cu) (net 2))
 (segment (start 59.055 60.96) (end 60.96 60.96) (width 0.635) (layer B.Cu) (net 2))
 (segment (start 67.405 85.09) (end 67.405 83.915) (width 0.635) (layer B.Cu) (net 2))
 (segment (start 66.04 82.55) (end 66.04 80.01) (width 0.635) (layer B.Cu) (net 2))
 (segment (start 67.405 83.915) (end 66.04 82.55) (width 0.635) (layer B.Cu) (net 2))
 (segment (start 61.69 85.09) (end 61.69 85.82) (width 0.635) (layer B.Cu) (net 2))
 (segment (start 61.69 85.82) (end 62.865 86.995) (width 0.635) (layer B.Cu) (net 2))
 (segment (start 62.865 86.995) (end 66.675 86.995) (width 0.635) (layer B.Cu) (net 2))
 (segment (start 67.405 86.265) (end 67.405 85.09) (width 0.635) (layer B.Cu) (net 2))
 (segment (start 66.675 86.995) (end 67.405 86.265) (width 0.635) (layer B.Cu) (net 2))
 (segment (start 66.04 60.96) (end 68.58 60.96) (width 0.635) (layer B.Cu) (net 2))
 (segment (start 83.185 88.9) (end 93.98 88.9) (width 0.635) (layer B.Cu) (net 1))
 (segment (start 80.645 86.36) (end 83.185 88.9) (width 0.635) (layer B.Cu) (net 1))
 (segment (start 107.95 79.375) (end 107.95 78.105) (width 0.635) (layer B.Cu) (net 1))
 (segment (start 100.965 86.36) (end 107.95 79.375) (width 0.635) (layer B.Cu) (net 1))
 (segment (start 107.95 78.105) (end 107.95 62.865) (width 0.635) (layer B.Cu) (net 1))
 (segment (start 95.885 53.34) (end 95.885 54.61) (width 0.635) (layer B.Cu) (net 1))
 (segment (start 82.55 52.705) (end 95.25 52.705) (width 0.635) (layer B.Cu) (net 1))
 (segment (start 95.25 52.705) (end 95.885 53.34) (width 0.635) (layer B.Cu) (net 1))
 (segment (start 80.645 53.34) (end 81.28 52.705) (width 0.635) (layer B.Cu) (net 1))
 (segment (start 81.28 52.705) (end 82.55 52.705) (width 0.635) (layer B.Cu) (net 1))
 (segment (start 80.645 53.34) (end 80.01 52.705) (width 0.635) (layer B.Cu) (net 1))
 (segment (start 80.645 54.61) (end 80.645 53.34) (width 0.635) (layer B.Cu) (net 1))
 (segment (start 80.01 52.705) (end 81.28 52.705) (width 0.635) (layer B.Cu) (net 1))
 (segment (start 98.425 88.9) (end 100.965 86.36) (width 0.635) (layer B.Cu) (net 1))
 (segment (start 95.885 86.36) (end 95.885 88.265) (width 0.635) (layer B.Cu) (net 1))
 (segment (start 93.98 88.9) (end 95.25 88.9) (width 0.635) (layer B.Cu) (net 1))
 (segment (start 95.885 88.265) (end 96.52 88.9) (width 0.635) (layer B.Cu) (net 1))
 (segment (start 96.52 88.9) (end 98.425 88.9) (width 0.635) (layer B.Cu) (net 1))
 (segment (start 95.25 88.9) (end 96.52 88.9) (width 0.635) (layer B.Cu) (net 1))
 (segment (start 95.885 53.34) (end 96.52 52.705) (width 0.635) (layer B.Cu) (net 1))
 (segment (start 96.52 52.705) (end 95.25 52.705) (width 0.635) (layer B.Cu) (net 1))
 (segment (start 95.885 88.265) (end 95.25 88.9) (width 0.635) (layer B.Cu) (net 1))
 (segment (start 96.52 52.705) (end 99.06 52.705) (width 0.635) (layer B.Cu) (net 1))
 (segment (start 107.95 61.595) (end 107.95 62.865) (width 0.635) (layer B.Cu) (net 1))
 (segment (start 99.06 52.705) (end 107.95 61.595) (width 0.635) (layer B.Cu) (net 1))
 (segment (start 71.755 57.785) (end 73.66 59.69) (width 0.635) (layer B.Cu) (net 1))
 (segment (start 71.12 57.785) (end 71.755 57.785) (width 0.635) (layer B.Cu) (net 1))
 (segment (start 73.66 59.69) (end 73.66 57.785) (width 0.635) (layer B.Cu) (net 1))
 (segment (start 73.66 60.96) (end 73.66 59.69) (width 0.635) (layer B.Cu) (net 1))
 (segment (start 71.755 57.785) (end 73.66 55.88) (width 0.635) (layer B.Cu) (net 1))
 (segment (start 73.66 57.785) (end 73.66 55.88) (width 0.635) (layer B.Cu) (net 1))
 (segment (start 76.835 52.705) (end 80.01 52.705) (width 0.635) (layer B.Cu) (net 1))
 (segment (start 73.66 55.88) (end 76.835 52.705) (width 0.635) (layer B.Cu) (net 1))
 (segment (start 66.48 54.61) (end 66.48 56.32) (width 0.635) (layer B.Cu) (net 1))
 (segment (start 67.945 57.785) (end 71.12 57.785) (width 0.635) (layer B.Cu) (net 1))
 (segment (start 66.48 56.32) (end 67.945 57.785) (width 0.635) (layer B.Cu) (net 1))
 (segment (start 73.66 60.96) (end 73.66 59.69) (width 0.635) (layer F.Cu) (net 1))
 (segment (start 73.66 59.69) (end 71.755 57.785) (width 0.635) (layer F.Cu) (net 1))
 (segment (start 71.755 57.785) (end 67.945 57.785) (width 0.635) (layer F.Cu) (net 1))
 (segment (start 66.48 56.32) (end 66.48 54.61) (width 0.635) (layer F.Cu) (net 1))
 (segment (start 67.945 57.785) (end 66.48 56.32) (width 0.635) (layer F.Cu) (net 1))
 (segment (start 73.66 64.77) (end 73.66 60.96) (width 0.635) (layer B.Cu) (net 1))
 (segment (start 73.66 60.96) (end 71.12 60.96) (width 0.635) (layer B.Cu) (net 1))
 (segment (start 81.28 57.785) (end 78.105 54.61) (width 0.635) (layer B.Cu) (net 17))
 (segment (start 86.36 57.785) (end 81.28 57.785) (width 0.635) (layer B.Cu) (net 17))
 (segment (start 93.345 64.77) (end 86.36 57.785) (width 0.635) (layer B.Cu) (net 17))
 (segment (start 93.345 60.96) (end 93.345 54.61) (width 0.635) (layer B.Cu) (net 18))
 (segment (start 93.345 68.58) (end 99.06 62.865) (width 0.635) (layer B.Cu) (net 16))
 (segment (start 99.06 62.865) (end 105.41 62.865) (width 0.635) (layer B.Cu) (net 16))
 (segment (start 93.345 72.39) (end 99.06 78.105) (width 0.635) (layer B.Cu) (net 14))
 (segment (start 99.06 78.105) (end 105.41 78.105) (width 0.635) (layer B.Cu) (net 14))
 (segment (start 93.345 80.01) (end 93.345 86.36) (width 0.635) (layer B.Cu) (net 11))
 (segment (start 85.725 83.82) (end 93.345 76.2) (width 0.635) (layer B.Cu) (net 12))
 (segment (start 80.01 83.82) (end 85.725 83.82) (width 0.635) (layer B.Cu) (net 12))
 (segment (start 78.105 85.725) (end 80.01 83.82) (width 0.635) (layer B.Cu) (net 12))
 (segment (start 78.105 86.36) (end 78.105 85.725) (width 0.635) (layer B.Cu) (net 12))
 (segment (start 64.48 56.17) (end 64.48 54.61) (width 0.635) (layer B.Cu) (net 3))
 (segment (start 56.515 60.96) (end 59.69 57.785) (width 0.635) (layer B.Cu) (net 3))
 (segment (start 59.69 57.785) (end 62.865 57.785) (width 0.635) (layer B.Cu) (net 3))
 (segment (start 62.865 57.785) (end 64.48 56.17) (width 0.635) (layer B.Cu) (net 3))
 (segment (start 53.34 60.96) (end 56.515 60.96) (width 0.635) (layer B.Cu) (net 3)))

